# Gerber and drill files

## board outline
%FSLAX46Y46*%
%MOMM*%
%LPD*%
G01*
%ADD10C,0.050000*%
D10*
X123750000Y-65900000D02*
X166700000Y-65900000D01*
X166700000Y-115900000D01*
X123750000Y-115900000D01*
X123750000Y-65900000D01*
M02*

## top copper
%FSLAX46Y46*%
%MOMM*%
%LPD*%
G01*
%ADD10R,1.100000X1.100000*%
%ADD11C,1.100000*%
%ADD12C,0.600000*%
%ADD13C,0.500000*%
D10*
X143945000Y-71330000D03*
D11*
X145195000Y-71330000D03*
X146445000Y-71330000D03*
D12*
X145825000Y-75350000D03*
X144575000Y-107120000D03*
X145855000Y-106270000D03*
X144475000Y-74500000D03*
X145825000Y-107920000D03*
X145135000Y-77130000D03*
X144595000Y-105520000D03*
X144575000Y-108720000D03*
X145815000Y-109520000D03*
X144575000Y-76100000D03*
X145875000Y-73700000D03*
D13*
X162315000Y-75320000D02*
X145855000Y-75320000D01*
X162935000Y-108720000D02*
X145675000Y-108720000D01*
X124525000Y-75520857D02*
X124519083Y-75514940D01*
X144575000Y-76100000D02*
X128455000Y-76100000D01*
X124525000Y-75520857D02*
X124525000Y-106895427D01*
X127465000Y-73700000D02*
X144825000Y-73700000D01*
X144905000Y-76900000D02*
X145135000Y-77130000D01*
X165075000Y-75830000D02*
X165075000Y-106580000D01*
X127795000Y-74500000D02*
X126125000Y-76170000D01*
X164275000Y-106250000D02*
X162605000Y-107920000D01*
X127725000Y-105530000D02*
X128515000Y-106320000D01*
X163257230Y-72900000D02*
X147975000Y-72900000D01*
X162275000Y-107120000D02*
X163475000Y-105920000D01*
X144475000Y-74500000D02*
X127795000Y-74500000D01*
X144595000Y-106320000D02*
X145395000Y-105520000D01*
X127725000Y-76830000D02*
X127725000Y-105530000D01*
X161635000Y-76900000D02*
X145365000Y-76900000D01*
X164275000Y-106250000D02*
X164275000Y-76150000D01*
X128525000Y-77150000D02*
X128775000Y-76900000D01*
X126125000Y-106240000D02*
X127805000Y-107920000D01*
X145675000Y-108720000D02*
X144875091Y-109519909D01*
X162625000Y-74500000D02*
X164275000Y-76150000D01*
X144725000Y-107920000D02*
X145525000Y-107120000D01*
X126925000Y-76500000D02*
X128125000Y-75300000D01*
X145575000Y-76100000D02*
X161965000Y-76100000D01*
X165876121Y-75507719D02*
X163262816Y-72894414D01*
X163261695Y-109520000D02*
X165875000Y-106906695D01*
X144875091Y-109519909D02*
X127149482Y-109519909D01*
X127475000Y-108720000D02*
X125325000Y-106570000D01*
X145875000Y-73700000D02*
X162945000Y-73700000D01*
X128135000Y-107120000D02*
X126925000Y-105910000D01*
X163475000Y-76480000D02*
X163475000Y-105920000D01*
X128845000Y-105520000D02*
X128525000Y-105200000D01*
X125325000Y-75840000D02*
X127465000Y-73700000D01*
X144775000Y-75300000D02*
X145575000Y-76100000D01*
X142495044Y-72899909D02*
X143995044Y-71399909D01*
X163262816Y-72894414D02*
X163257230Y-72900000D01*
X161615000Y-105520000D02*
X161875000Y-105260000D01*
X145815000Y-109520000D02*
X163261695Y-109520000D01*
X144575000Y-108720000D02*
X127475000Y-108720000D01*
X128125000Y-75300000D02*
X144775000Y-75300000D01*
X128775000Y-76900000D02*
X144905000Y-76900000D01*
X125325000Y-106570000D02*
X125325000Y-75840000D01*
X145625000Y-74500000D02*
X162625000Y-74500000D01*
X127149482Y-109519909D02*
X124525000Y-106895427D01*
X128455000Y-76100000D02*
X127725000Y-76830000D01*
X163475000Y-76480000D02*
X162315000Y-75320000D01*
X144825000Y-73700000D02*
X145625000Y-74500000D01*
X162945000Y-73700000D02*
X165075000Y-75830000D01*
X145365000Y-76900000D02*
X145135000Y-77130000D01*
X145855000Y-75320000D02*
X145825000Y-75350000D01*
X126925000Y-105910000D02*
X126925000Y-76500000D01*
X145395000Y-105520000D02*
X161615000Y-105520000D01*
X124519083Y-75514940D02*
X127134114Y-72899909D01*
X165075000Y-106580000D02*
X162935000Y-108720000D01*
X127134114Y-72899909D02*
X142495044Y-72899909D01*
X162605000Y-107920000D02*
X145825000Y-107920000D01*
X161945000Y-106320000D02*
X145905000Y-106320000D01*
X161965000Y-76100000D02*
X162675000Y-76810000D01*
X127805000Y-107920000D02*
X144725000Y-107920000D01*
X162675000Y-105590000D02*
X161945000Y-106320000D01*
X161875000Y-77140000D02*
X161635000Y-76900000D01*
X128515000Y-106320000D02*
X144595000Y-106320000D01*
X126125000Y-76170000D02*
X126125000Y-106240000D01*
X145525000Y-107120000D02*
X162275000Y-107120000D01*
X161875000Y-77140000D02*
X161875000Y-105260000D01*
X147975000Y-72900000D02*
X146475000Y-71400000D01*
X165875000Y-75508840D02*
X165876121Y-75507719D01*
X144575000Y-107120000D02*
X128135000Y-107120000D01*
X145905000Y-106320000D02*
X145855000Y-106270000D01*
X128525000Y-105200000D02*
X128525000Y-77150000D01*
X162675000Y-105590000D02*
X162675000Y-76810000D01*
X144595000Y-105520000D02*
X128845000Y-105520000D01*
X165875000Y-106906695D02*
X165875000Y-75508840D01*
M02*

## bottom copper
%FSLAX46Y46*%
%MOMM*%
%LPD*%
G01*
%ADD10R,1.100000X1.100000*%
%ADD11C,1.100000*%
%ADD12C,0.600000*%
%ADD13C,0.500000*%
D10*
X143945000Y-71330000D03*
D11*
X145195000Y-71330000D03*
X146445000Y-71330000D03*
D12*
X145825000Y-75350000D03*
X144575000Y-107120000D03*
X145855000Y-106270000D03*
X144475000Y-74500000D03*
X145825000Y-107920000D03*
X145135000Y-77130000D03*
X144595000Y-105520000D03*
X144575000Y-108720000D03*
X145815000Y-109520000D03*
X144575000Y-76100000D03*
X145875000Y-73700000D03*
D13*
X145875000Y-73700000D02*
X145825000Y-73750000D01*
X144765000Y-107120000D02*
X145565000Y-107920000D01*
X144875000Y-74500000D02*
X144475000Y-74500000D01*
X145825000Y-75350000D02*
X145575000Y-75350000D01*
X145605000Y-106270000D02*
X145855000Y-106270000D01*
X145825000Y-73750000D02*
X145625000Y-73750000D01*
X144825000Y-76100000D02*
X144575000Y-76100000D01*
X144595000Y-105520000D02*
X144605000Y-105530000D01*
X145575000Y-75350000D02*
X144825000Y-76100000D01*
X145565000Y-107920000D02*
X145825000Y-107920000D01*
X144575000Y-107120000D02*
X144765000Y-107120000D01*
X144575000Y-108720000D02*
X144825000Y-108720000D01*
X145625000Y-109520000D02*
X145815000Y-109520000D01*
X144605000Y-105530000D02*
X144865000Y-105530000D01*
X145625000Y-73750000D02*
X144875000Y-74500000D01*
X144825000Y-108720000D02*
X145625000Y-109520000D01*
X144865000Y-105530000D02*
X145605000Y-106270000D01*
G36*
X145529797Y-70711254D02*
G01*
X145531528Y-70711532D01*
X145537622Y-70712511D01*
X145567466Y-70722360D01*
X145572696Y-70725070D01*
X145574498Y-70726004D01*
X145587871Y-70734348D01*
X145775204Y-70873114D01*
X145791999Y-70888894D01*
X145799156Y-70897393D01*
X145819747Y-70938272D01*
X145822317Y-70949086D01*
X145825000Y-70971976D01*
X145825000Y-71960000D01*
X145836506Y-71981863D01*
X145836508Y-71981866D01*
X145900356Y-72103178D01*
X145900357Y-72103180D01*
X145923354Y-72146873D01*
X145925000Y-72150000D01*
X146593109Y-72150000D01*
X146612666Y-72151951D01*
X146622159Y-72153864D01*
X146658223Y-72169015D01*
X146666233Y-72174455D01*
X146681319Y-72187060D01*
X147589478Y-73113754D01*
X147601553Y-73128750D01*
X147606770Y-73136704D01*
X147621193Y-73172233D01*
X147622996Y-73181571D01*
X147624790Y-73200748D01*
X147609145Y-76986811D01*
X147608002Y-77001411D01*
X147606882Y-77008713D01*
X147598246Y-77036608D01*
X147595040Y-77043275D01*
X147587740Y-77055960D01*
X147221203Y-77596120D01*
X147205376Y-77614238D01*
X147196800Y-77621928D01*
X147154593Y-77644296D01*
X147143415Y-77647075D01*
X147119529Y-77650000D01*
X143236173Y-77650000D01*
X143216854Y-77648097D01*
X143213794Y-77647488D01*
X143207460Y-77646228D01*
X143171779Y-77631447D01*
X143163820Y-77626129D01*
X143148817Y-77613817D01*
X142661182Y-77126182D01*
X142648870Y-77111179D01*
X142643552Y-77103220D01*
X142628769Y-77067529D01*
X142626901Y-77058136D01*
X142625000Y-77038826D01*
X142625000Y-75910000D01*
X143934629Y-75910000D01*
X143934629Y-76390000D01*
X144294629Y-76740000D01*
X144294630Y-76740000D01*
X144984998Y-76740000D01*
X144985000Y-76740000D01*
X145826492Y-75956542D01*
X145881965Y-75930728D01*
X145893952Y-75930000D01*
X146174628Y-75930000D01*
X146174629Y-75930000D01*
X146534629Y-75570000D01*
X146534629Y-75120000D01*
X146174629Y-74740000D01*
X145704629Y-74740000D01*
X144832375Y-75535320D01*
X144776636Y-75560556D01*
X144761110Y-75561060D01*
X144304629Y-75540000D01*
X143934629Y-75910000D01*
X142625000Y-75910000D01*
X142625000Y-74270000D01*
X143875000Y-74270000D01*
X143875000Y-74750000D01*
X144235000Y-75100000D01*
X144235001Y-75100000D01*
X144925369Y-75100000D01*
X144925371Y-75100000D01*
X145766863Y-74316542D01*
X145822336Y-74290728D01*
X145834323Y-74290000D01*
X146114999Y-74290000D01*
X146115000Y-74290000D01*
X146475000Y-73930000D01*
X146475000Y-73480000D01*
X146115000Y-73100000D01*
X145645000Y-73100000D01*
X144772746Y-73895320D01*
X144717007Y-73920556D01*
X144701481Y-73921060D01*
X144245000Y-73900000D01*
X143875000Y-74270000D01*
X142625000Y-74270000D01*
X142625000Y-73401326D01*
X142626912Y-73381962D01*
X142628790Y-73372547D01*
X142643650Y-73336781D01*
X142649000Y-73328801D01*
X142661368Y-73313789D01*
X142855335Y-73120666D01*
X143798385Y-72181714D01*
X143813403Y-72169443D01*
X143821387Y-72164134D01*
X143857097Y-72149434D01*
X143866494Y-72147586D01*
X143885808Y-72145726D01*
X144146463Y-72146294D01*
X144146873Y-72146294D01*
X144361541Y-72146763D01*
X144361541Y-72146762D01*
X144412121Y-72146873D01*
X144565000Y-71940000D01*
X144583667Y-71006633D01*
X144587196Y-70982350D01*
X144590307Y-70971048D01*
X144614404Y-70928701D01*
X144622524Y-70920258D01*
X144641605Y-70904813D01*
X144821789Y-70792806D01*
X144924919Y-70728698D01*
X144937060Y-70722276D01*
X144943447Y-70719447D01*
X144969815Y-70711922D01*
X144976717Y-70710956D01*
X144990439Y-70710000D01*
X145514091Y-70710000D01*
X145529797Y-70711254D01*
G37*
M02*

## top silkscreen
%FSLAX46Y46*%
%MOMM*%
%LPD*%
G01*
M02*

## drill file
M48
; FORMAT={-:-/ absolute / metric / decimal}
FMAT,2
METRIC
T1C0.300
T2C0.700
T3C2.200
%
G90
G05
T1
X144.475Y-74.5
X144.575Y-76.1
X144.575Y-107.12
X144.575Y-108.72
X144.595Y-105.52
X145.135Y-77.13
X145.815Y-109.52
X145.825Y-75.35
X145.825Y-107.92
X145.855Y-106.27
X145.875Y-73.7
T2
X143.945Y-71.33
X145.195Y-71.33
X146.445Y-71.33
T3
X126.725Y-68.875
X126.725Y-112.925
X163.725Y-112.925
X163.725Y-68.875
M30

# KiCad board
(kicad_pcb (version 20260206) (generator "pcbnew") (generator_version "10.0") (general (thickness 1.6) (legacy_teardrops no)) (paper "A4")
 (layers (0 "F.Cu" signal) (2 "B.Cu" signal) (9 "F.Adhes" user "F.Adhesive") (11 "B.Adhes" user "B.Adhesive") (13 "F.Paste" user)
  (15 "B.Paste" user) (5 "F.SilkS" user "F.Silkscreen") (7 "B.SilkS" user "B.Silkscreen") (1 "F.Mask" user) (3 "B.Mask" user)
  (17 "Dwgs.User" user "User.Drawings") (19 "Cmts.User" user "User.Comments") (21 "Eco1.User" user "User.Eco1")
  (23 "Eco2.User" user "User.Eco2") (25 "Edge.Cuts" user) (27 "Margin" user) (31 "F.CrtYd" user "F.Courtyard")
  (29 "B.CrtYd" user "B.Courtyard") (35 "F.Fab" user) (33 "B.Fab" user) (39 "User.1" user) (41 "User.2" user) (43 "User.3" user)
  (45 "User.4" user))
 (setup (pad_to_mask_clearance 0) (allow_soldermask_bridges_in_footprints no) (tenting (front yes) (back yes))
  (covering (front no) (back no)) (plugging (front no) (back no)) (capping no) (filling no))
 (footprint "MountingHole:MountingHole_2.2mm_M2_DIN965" (layer "F.Cu") (at 126.725 112.925)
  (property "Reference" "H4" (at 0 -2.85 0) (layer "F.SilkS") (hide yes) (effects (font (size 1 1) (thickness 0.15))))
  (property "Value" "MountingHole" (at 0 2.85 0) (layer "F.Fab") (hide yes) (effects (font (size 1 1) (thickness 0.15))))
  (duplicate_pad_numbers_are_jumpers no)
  (pad "" np_thru_hole circle (at 0 0) (size 2.2 2.2) (drill 2.2) (layers "*.Cu" "*.Mask")))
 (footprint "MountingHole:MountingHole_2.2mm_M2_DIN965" (layer "F.Cu") (at 163.725 68.875)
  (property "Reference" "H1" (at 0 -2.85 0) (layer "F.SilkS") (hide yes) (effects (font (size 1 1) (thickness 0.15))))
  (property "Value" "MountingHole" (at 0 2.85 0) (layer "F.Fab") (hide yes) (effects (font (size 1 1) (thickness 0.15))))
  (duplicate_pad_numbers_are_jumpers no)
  (pad "" np_thru_hole circle (at 0 0) (size 2.2 2.2) (drill 2.2) (layers "*.Cu" "*.Mask")))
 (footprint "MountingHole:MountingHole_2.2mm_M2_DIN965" (layer "F.Cu") (at 163.724986 112.924986)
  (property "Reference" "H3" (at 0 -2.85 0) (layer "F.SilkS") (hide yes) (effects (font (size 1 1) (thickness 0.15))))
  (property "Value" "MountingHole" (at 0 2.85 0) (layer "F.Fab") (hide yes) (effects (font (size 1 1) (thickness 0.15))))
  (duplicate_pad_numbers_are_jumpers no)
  (pad "" np_thru_hole circle (at 0 0) (size 2.2 2.2) (drill 2.2) (layers "*.Cu" "*.Mask")))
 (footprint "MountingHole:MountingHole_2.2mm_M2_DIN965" (layer "F.Cu") (at 126.725 68.875)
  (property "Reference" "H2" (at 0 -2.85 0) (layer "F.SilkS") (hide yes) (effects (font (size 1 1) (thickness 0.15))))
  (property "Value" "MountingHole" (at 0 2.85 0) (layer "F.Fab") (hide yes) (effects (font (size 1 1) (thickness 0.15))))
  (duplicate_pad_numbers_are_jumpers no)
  (pad "" np_thru_hole circle (at 0 0) (size 2.2 2.2) (drill 2.2) (layers "*.Cu" "*.Mask")))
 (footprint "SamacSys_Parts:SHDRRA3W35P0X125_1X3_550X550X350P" (layer "B.Cu") (at 143.945 71.33 180)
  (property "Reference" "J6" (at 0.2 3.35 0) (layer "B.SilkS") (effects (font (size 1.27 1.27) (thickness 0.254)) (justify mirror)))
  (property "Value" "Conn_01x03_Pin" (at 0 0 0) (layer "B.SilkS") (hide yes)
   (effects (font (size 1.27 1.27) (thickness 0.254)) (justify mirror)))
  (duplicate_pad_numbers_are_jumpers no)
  (pad "1" thru_hole rect (at 0 0 180) (size 1.1 1.1) (drill 0.7) (layers "*.Cu" "*.Mask") (remove_unused_layers no) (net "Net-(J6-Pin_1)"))
  (pad "2" thru_hole circle (at -1.25 0 180) (size 1.1 1.1) (drill 0.7) (layers "*.Cu" "*.Mask") (remove_unused_layers no)
   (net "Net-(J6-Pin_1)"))
  (pad "3" thru_hole circle (at -2.5 0 180) (size 1.1 1.1) (drill 0.7) (layers "*.Cu" "*.Mask") (remove_unused_layers no)
   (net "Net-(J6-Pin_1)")))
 (gr_rect (start 123.75 65.9) (end 166.7 115.9) (stroke (width 0.05) (type default)) (fill no) (layer "Edge.Cuts"))
 (segment (start 162.315 75.32) (end 145.855 75.32) (width 0.5) (layer "F.Cu") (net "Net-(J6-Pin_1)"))
 (segment (start 162.935 108.72) (end 145.675 108.72) (width 0.5) (layer "F.Cu") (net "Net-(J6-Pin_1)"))
 (segment (start 124.525 75.520857) (end 124.519083 75.51494) (width 0.5) (layer "F.Cu") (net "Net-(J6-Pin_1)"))
 (segment (start 144.575 76.1) (end 128.455 76.1) (width 0.5) (layer "F.Cu") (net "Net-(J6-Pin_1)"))
 (segment (start 124.525 75.520857) (end 124.525 106.895427) (width 0.5) (layer "F.Cu") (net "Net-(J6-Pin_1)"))
 (segment (start 127.465 73.7) (end 144.825 73.7) (width 0.5) (layer "F.Cu") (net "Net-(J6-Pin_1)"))
 (segment (start 144.905 76.9) (end 145.135 77.13) (width 0.5) (layer "F.Cu") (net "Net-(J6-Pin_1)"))
 (segment (start 165.075 75.83) (end 165.075 106.58) (width 0.5) (layer "F.Cu") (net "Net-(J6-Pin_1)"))
 (segment (start 127.795 74.5) (end 126.125 76.17) (width 0.5) (layer "F.Cu") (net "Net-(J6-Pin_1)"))
 (segment (start 164.275 106.25) (end 162.605 107.92) (width 0.5) (layer "F.Cu") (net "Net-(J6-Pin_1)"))
 (segment (start 127.725 105.53) (end 128.515 106.32) (width 0.5) (layer "F.Cu") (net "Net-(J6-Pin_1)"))
 (segment (start 163.25723 72.9) (end 147.975 72.9) (width 0.5) (layer "F.Cu") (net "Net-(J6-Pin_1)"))
 (segment (start 162.275 107.12) (end 163.475 105.92) (width 0.5) (layer "F.Cu") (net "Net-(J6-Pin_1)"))
 (segment (start 144.475 74.5) (end 127.795 74.5) (width 0.5) (layer "F.Cu") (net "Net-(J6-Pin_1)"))
 (segment (start 144.595 106.32) (end 145.395 105.52) (width 0.5) (layer "F.Cu") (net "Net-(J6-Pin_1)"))
 (segment (start 127.725 76.83) (end 127.725 105.53) (width 0.5) (layer "F.Cu") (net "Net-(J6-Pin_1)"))
 (segment (start 161.635 76.9) (end 145.365 76.9) (width 0.5) (layer "F.Cu") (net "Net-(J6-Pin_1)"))
 (segment (start 164.275 106.25) (end 164.275 76.15) (width 0.5) (layer "F.Cu") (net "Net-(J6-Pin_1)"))
 (segment (start 128.525 77.15) (end 128.775 76.9) (width 0.5) (layer "F.Cu") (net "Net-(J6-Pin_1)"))
 (segment (start 126.125 106.24) (end 127.805 107.92) (width 0.5) (layer "F.Cu") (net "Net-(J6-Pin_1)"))
 (segment (start 145.675 108.72) (end 144.875091 109.519909) (width 0.5) (layer "F.Cu") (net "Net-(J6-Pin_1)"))
 (segment (start 162.625 74.5) (end 164.275 76.15) (width 0.5) (layer "F.Cu") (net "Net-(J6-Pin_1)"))
 (segment (start 144.725 107.92) (end 145.525 107.12) (width 0.5) (layer "F.Cu") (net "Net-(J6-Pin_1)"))
 (segment (start 126.925 76.5) (end 128.125 75.3) (width 0.5) (layer "F.Cu") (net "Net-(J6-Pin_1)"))
 (segment (start 145.575 76.1) (end 161.965 76.1) (width 0.5) (layer "F.Cu") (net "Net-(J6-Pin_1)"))
 (segment (start 165.876121 75.507719) (end 163.262816 72.894414) (width 0.5) (layer "F.Cu") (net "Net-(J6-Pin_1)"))
 (segment (start 163.261695 109.52) (end 165.875 106.906695) (width 0.5) (layer "F.Cu") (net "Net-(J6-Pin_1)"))
 (segment (start 144.875091 109.519909) (end 127.149482 109.519909) (width 0.5) (layer "F.Cu") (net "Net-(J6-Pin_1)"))
 (segment (start 127.475 108.72) (end 125.325 106.57) (width 0.5) (layer "F.Cu") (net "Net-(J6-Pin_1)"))
 (segment (start 145.875 73.7) (end 162.945 73.7) (width 0.5) (layer "F.Cu") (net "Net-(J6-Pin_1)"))
 (segment (start 128.135 107.12) (end 126.925 105.91) (width 0.5) (layer "F.Cu") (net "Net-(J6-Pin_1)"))
 (segment (start 163.475 76.48) (end 163.475 105.92) (width 0.5) (layer "F.Cu") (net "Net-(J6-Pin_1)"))
 (segment (start 128.845 105.52) (end 128.525 105.2) (width 0.5) (layer "F.Cu") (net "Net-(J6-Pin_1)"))
 (segment (start 125.325 75.84) (end 127.465 73.7) (width 0.5) (layer "F.Cu") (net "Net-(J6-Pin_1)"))
 (segment (start 144.775 75.3) (end 145.575 76.1) (width 0.5) (layer "F.Cu") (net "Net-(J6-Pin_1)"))
 (segment (start 142.495044 72.899909) (end 143.995044 71.399909) (width 0.5) (layer "F.Cu") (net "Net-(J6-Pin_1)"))
 (segment (start 163.262816 72.894414) (end 163.25723 72.9) (width 0.5) (layer "F.Cu") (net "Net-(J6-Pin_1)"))
 (segment (start 161.615 105.52) (end 161.875 105.26) (width 0.5) (layer "F.Cu") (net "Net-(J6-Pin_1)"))
 (segment (start 145.815 109.52) (end 163.261695 109.52) (width 0.5) (layer "F.Cu") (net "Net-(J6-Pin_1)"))
 (segment (start 144.575 108.72) (end 127.475 108.72) (width 0.5) (layer "F.Cu") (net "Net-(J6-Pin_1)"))
 (segment (start 128.125 75.3) (end 144.775 75.3) (width 0.5) (layer "F.Cu") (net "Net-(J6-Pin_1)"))
 (segment (start 128.775 76.9) (end 144.905 76.9) (width 0.5) (layer "F.Cu") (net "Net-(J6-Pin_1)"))
 (segment (start 125.325 106.57) (end 125.325 75.84) (width 0.5) (layer "F.Cu") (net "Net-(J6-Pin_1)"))
 (segment (start 145.625 74.5) (end 162.625 74.5) (width 0.5) (layer "F.Cu") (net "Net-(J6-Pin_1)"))
 (segment (start 127.149482 109.519909) (end 124.525 106.895427) (width 0.5) (layer "F.Cu") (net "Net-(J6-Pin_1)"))
 (segment (start 128.455 76.1) (end 127.725 76.83) (width 0.5) (layer "F.Cu") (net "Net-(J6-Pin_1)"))
 (segment (start 163.475 76.48) (end 162.315 75.32) (width 0.5) (layer "F.Cu") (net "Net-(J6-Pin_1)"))
 (segment (start 144.825 73.7) (end 145.625 74.5) (width 0.5) (layer "F.Cu") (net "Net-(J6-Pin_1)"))
 (segment (start 162.945 73.7) (end 165.075 75.83) (width 0.5) (layer "F.Cu") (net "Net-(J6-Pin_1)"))
 (segment (start 145.365 76.9) (end 145.135 77.13) (width 0.5) (layer "F.Cu") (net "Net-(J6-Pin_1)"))
 (segment (start 145.855 75.32) (end 145.825 75.35) (width 0.5) (layer "F.Cu") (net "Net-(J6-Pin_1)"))
 (segment (start 126.925 105.91) (end 126.925 76.5) (width 0.5) (layer "F.Cu") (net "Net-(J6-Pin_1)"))
 (segment (start 145.395 105.52) (end 161.615 105.52) (width 0.5) (layer "F.Cu") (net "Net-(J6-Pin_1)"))
 (segment (start 124.519083 75.51494) (end 127.134114 72.899909) (width 0.5) (layer "F.Cu") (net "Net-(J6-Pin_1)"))
 (segment (start 165.075 106.58) (end 162.935 108.72) (width 0.5) (layer "F.Cu") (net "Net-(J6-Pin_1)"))
 (segment (start 127.134114 72.899909) (end 142.495044 72.899909) (width 0.5) (layer "F.Cu") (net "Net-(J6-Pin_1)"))
 (segment (start 162.605 107.92) (end 145.825 107.92) (width 0.5) (layer "F.Cu") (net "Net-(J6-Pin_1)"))
 (segment (start 161.945 106.32) (end 145.905 106.32) (width 0.5) (layer "F.Cu") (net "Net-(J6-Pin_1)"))
 (segment (start 161.965 76.1) (end 162.675 76.81) (width 0.5) (layer "F.Cu") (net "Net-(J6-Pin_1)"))
 (segment (start 127.805 107.92) (end 144.725 107.92) (width 0.5) (layer "F.Cu") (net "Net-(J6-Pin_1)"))
 (segment (start 162.675 105.59) (end 161.945 106.32) (width 0.5) (layer "F.Cu") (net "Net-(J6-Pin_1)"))
 (segment (start 161.875 77.14) (end 161.635 76.9) (width 0.5) (layer "F.Cu") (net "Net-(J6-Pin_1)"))
 (segment (start 128.515 106.32) (end 144.595 106.32) (width 0.5) (layer "F.Cu") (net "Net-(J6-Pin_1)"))
 (segment (start 126.125 76.17) (end 126.125 106.24) (width 0.5) (layer "F.Cu") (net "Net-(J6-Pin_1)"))
 (segment (start 145.525 107.12) (end 162.275 107.12) (width 0.5) (layer "F.Cu") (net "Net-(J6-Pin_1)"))
 (segment (start 161.875 77.14) (end 161.875 105.26) (width 0.5) (layer "F.Cu") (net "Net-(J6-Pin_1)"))
 (segment (start 147.975 72.9) (end 146.475 71.4) (width 0.5) (layer "F.Cu") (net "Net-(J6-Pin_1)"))
 (segment (start 165.875 75.50884) (end 165.876121 75.507719) (width 0.5) (layer "F.Cu") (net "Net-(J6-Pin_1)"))
 (segment (start 144.575 107.12) (end 128.135 107.12) (width 0.5) (layer "F.Cu") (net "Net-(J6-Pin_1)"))
 (segment (start 145.905 106.32) (end 145.855 106.27) (width 0.5) (layer "F.Cu") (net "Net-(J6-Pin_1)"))
 (segment (start 128.525 105.2) (end 128.525 77.15) (width 0.5) (layer "F.Cu") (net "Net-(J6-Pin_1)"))
 (segment (start 162.675 105.59) (end 162.675 76.81) (width 0.5) (layer "F.Cu") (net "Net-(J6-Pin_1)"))
 (segment (start 144.595 105.52) (end 128.845 105.52) (width 0.5) (layer "F.Cu") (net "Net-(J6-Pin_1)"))
 (segment (start 165.875 106.906695) (end 165.875 75.50884) (width 0.5) (layer "F.Cu") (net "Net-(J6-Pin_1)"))
 (via (at 145.825 75.35) (size 0.6) (drill 0.3) (layers "F.Cu" "B.Cu") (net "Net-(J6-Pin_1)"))
 (via (at 144.575 107.12) (size 0.6) (drill 0.3) (layers "F.Cu" "B.Cu") (free yes) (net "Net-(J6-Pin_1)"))
 (via (at 145.855 106.27) (size 0.6) (drill 0.3) (layers "F.Cu" "B.Cu") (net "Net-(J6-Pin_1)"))
 (via (at 144.475 74.5) (size 0.6) (drill 0.3) (layers "F.Cu" "B.Cu") (free yes) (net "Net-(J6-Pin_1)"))
 (via (at 145.825 107.92) (size 0.6) (drill 0.3) (layers "F.Cu" "B.Cu") (free yes) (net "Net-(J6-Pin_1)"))
 (via (at 145.135 77.13) (size 0.6) (drill 0.3) (layers "F.Cu" "B.Cu") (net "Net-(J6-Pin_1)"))
 (via (at 144.595 105.52) (size 0.6) (drill 0.3) (layers "F.Cu" "B.Cu") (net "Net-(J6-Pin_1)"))
 (via (at 144.575 108.72) (size 0.6) (drill 0.3) (layers "F.Cu" "B.Cu") (free yes) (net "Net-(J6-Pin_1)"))
 (via (at 145.815 109.52) (size 0.6) (drill 0.3) (layers "F.Cu" "B.Cu") (free yes) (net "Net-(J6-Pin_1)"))
 (via (at 144.575 76.1) (size 0.6) (drill 0.3) (layers "F.Cu" "B.Cu") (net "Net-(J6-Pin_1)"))
 (via (at 145.875 73.7) (size 0.6) (drill 0.3) (layers "F.Cu" "B.Cu") (free yes) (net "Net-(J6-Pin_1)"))
 (segment (start 145.875 73.7) (end 145.825 73.75) (width 0.5) (layer "B.Cu") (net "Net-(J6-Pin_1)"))
 (segment (start 144.765 107.12) (end 145.565 107.92) (width 0.5) (layer "B.Cu") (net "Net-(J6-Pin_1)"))
 (segment (start 144.875 74.5) (end 144.475 74.5) (width 0.5) (layer "B.Cu") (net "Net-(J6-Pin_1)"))
 (segment (start 145.825 75.35) (end 145.575 75.35) (width 0.5) (layer "B.Cu") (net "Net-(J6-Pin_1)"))
 (segment (start 145.605 106.27) (end 145.855 106.27) (width 0.5) (layer "B.Cu") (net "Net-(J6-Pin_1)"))
 (segment (start 145.825 73.75) (end 145.625 73.75) (width 0.5) (layer "B.Cu") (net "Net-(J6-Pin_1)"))
 (segment (start 144.825 76.1) (end 144.575 76.1) (width 0.5) (layer "B.Cu") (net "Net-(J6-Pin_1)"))
 (segment (start 144.595 105.52) (end 144.605 105.53) (width 0.5) (layer "B.Cu") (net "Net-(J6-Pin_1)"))
 (segment (start 145.575 75.35) (end 144.825 76.1) (width 0.5) (layer "B.Cu") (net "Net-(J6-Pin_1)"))
 (segment (start 145.565 107.92) (end 145.825 107.92) (width 0.5) (layer "B.Cu") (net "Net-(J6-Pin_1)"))
 (segment (start 144.575 107.12) (end 144.765 107.12) (width 0.5) (layer "B.Cu") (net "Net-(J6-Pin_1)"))
 (segment (start 144.575 108.72) (end 144.825 108.72) (width 0.5) (layer "B.Cu") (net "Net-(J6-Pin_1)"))
 (segment (start 145.625 109.52) (end 145.815 109.52) (width 0.5) (layer "B.Cu") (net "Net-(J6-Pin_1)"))
 (segment (start 144.605 105.53) (end 144.865 105.53) (width 0.5) (layer "B.Cu") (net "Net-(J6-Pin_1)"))
 (segment (start 145.625 73.75) (end 144.875 74.5) (width 0.5) (layer "B.Cu") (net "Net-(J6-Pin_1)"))
 (segment (start 144.825 108.72) (end 145.625 109.52) (width 0.5) (layer "B.Cu") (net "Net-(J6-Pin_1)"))
 (segment (start 144.865 105.53) (end 145.605 106.27) (width 0.5) (layer "B.Cu") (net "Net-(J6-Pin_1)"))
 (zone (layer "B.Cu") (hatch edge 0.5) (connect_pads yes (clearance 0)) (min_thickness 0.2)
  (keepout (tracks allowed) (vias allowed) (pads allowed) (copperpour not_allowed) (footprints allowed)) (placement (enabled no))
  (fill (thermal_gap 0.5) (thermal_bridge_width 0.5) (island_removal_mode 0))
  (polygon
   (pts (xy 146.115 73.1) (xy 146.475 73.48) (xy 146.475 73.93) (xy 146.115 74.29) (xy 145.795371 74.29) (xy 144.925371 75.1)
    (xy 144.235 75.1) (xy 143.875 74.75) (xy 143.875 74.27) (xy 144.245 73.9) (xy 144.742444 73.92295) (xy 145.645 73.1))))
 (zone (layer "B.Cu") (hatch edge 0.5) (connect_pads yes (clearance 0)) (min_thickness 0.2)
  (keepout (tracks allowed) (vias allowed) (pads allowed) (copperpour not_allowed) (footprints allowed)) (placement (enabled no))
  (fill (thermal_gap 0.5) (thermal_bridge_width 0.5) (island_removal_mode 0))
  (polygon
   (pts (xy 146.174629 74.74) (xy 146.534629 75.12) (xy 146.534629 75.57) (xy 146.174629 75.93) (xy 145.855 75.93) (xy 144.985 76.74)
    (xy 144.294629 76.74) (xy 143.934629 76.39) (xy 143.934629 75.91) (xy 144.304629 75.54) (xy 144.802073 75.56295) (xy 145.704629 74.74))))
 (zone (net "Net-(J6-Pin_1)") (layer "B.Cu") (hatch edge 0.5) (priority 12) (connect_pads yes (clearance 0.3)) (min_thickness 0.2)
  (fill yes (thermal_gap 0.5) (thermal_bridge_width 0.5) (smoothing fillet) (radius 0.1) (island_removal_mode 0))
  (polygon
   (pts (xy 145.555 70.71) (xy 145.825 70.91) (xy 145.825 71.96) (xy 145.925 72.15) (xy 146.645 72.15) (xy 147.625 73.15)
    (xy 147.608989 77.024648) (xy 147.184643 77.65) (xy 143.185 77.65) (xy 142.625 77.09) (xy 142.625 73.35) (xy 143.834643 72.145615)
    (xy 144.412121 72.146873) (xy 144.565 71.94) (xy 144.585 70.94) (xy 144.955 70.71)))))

